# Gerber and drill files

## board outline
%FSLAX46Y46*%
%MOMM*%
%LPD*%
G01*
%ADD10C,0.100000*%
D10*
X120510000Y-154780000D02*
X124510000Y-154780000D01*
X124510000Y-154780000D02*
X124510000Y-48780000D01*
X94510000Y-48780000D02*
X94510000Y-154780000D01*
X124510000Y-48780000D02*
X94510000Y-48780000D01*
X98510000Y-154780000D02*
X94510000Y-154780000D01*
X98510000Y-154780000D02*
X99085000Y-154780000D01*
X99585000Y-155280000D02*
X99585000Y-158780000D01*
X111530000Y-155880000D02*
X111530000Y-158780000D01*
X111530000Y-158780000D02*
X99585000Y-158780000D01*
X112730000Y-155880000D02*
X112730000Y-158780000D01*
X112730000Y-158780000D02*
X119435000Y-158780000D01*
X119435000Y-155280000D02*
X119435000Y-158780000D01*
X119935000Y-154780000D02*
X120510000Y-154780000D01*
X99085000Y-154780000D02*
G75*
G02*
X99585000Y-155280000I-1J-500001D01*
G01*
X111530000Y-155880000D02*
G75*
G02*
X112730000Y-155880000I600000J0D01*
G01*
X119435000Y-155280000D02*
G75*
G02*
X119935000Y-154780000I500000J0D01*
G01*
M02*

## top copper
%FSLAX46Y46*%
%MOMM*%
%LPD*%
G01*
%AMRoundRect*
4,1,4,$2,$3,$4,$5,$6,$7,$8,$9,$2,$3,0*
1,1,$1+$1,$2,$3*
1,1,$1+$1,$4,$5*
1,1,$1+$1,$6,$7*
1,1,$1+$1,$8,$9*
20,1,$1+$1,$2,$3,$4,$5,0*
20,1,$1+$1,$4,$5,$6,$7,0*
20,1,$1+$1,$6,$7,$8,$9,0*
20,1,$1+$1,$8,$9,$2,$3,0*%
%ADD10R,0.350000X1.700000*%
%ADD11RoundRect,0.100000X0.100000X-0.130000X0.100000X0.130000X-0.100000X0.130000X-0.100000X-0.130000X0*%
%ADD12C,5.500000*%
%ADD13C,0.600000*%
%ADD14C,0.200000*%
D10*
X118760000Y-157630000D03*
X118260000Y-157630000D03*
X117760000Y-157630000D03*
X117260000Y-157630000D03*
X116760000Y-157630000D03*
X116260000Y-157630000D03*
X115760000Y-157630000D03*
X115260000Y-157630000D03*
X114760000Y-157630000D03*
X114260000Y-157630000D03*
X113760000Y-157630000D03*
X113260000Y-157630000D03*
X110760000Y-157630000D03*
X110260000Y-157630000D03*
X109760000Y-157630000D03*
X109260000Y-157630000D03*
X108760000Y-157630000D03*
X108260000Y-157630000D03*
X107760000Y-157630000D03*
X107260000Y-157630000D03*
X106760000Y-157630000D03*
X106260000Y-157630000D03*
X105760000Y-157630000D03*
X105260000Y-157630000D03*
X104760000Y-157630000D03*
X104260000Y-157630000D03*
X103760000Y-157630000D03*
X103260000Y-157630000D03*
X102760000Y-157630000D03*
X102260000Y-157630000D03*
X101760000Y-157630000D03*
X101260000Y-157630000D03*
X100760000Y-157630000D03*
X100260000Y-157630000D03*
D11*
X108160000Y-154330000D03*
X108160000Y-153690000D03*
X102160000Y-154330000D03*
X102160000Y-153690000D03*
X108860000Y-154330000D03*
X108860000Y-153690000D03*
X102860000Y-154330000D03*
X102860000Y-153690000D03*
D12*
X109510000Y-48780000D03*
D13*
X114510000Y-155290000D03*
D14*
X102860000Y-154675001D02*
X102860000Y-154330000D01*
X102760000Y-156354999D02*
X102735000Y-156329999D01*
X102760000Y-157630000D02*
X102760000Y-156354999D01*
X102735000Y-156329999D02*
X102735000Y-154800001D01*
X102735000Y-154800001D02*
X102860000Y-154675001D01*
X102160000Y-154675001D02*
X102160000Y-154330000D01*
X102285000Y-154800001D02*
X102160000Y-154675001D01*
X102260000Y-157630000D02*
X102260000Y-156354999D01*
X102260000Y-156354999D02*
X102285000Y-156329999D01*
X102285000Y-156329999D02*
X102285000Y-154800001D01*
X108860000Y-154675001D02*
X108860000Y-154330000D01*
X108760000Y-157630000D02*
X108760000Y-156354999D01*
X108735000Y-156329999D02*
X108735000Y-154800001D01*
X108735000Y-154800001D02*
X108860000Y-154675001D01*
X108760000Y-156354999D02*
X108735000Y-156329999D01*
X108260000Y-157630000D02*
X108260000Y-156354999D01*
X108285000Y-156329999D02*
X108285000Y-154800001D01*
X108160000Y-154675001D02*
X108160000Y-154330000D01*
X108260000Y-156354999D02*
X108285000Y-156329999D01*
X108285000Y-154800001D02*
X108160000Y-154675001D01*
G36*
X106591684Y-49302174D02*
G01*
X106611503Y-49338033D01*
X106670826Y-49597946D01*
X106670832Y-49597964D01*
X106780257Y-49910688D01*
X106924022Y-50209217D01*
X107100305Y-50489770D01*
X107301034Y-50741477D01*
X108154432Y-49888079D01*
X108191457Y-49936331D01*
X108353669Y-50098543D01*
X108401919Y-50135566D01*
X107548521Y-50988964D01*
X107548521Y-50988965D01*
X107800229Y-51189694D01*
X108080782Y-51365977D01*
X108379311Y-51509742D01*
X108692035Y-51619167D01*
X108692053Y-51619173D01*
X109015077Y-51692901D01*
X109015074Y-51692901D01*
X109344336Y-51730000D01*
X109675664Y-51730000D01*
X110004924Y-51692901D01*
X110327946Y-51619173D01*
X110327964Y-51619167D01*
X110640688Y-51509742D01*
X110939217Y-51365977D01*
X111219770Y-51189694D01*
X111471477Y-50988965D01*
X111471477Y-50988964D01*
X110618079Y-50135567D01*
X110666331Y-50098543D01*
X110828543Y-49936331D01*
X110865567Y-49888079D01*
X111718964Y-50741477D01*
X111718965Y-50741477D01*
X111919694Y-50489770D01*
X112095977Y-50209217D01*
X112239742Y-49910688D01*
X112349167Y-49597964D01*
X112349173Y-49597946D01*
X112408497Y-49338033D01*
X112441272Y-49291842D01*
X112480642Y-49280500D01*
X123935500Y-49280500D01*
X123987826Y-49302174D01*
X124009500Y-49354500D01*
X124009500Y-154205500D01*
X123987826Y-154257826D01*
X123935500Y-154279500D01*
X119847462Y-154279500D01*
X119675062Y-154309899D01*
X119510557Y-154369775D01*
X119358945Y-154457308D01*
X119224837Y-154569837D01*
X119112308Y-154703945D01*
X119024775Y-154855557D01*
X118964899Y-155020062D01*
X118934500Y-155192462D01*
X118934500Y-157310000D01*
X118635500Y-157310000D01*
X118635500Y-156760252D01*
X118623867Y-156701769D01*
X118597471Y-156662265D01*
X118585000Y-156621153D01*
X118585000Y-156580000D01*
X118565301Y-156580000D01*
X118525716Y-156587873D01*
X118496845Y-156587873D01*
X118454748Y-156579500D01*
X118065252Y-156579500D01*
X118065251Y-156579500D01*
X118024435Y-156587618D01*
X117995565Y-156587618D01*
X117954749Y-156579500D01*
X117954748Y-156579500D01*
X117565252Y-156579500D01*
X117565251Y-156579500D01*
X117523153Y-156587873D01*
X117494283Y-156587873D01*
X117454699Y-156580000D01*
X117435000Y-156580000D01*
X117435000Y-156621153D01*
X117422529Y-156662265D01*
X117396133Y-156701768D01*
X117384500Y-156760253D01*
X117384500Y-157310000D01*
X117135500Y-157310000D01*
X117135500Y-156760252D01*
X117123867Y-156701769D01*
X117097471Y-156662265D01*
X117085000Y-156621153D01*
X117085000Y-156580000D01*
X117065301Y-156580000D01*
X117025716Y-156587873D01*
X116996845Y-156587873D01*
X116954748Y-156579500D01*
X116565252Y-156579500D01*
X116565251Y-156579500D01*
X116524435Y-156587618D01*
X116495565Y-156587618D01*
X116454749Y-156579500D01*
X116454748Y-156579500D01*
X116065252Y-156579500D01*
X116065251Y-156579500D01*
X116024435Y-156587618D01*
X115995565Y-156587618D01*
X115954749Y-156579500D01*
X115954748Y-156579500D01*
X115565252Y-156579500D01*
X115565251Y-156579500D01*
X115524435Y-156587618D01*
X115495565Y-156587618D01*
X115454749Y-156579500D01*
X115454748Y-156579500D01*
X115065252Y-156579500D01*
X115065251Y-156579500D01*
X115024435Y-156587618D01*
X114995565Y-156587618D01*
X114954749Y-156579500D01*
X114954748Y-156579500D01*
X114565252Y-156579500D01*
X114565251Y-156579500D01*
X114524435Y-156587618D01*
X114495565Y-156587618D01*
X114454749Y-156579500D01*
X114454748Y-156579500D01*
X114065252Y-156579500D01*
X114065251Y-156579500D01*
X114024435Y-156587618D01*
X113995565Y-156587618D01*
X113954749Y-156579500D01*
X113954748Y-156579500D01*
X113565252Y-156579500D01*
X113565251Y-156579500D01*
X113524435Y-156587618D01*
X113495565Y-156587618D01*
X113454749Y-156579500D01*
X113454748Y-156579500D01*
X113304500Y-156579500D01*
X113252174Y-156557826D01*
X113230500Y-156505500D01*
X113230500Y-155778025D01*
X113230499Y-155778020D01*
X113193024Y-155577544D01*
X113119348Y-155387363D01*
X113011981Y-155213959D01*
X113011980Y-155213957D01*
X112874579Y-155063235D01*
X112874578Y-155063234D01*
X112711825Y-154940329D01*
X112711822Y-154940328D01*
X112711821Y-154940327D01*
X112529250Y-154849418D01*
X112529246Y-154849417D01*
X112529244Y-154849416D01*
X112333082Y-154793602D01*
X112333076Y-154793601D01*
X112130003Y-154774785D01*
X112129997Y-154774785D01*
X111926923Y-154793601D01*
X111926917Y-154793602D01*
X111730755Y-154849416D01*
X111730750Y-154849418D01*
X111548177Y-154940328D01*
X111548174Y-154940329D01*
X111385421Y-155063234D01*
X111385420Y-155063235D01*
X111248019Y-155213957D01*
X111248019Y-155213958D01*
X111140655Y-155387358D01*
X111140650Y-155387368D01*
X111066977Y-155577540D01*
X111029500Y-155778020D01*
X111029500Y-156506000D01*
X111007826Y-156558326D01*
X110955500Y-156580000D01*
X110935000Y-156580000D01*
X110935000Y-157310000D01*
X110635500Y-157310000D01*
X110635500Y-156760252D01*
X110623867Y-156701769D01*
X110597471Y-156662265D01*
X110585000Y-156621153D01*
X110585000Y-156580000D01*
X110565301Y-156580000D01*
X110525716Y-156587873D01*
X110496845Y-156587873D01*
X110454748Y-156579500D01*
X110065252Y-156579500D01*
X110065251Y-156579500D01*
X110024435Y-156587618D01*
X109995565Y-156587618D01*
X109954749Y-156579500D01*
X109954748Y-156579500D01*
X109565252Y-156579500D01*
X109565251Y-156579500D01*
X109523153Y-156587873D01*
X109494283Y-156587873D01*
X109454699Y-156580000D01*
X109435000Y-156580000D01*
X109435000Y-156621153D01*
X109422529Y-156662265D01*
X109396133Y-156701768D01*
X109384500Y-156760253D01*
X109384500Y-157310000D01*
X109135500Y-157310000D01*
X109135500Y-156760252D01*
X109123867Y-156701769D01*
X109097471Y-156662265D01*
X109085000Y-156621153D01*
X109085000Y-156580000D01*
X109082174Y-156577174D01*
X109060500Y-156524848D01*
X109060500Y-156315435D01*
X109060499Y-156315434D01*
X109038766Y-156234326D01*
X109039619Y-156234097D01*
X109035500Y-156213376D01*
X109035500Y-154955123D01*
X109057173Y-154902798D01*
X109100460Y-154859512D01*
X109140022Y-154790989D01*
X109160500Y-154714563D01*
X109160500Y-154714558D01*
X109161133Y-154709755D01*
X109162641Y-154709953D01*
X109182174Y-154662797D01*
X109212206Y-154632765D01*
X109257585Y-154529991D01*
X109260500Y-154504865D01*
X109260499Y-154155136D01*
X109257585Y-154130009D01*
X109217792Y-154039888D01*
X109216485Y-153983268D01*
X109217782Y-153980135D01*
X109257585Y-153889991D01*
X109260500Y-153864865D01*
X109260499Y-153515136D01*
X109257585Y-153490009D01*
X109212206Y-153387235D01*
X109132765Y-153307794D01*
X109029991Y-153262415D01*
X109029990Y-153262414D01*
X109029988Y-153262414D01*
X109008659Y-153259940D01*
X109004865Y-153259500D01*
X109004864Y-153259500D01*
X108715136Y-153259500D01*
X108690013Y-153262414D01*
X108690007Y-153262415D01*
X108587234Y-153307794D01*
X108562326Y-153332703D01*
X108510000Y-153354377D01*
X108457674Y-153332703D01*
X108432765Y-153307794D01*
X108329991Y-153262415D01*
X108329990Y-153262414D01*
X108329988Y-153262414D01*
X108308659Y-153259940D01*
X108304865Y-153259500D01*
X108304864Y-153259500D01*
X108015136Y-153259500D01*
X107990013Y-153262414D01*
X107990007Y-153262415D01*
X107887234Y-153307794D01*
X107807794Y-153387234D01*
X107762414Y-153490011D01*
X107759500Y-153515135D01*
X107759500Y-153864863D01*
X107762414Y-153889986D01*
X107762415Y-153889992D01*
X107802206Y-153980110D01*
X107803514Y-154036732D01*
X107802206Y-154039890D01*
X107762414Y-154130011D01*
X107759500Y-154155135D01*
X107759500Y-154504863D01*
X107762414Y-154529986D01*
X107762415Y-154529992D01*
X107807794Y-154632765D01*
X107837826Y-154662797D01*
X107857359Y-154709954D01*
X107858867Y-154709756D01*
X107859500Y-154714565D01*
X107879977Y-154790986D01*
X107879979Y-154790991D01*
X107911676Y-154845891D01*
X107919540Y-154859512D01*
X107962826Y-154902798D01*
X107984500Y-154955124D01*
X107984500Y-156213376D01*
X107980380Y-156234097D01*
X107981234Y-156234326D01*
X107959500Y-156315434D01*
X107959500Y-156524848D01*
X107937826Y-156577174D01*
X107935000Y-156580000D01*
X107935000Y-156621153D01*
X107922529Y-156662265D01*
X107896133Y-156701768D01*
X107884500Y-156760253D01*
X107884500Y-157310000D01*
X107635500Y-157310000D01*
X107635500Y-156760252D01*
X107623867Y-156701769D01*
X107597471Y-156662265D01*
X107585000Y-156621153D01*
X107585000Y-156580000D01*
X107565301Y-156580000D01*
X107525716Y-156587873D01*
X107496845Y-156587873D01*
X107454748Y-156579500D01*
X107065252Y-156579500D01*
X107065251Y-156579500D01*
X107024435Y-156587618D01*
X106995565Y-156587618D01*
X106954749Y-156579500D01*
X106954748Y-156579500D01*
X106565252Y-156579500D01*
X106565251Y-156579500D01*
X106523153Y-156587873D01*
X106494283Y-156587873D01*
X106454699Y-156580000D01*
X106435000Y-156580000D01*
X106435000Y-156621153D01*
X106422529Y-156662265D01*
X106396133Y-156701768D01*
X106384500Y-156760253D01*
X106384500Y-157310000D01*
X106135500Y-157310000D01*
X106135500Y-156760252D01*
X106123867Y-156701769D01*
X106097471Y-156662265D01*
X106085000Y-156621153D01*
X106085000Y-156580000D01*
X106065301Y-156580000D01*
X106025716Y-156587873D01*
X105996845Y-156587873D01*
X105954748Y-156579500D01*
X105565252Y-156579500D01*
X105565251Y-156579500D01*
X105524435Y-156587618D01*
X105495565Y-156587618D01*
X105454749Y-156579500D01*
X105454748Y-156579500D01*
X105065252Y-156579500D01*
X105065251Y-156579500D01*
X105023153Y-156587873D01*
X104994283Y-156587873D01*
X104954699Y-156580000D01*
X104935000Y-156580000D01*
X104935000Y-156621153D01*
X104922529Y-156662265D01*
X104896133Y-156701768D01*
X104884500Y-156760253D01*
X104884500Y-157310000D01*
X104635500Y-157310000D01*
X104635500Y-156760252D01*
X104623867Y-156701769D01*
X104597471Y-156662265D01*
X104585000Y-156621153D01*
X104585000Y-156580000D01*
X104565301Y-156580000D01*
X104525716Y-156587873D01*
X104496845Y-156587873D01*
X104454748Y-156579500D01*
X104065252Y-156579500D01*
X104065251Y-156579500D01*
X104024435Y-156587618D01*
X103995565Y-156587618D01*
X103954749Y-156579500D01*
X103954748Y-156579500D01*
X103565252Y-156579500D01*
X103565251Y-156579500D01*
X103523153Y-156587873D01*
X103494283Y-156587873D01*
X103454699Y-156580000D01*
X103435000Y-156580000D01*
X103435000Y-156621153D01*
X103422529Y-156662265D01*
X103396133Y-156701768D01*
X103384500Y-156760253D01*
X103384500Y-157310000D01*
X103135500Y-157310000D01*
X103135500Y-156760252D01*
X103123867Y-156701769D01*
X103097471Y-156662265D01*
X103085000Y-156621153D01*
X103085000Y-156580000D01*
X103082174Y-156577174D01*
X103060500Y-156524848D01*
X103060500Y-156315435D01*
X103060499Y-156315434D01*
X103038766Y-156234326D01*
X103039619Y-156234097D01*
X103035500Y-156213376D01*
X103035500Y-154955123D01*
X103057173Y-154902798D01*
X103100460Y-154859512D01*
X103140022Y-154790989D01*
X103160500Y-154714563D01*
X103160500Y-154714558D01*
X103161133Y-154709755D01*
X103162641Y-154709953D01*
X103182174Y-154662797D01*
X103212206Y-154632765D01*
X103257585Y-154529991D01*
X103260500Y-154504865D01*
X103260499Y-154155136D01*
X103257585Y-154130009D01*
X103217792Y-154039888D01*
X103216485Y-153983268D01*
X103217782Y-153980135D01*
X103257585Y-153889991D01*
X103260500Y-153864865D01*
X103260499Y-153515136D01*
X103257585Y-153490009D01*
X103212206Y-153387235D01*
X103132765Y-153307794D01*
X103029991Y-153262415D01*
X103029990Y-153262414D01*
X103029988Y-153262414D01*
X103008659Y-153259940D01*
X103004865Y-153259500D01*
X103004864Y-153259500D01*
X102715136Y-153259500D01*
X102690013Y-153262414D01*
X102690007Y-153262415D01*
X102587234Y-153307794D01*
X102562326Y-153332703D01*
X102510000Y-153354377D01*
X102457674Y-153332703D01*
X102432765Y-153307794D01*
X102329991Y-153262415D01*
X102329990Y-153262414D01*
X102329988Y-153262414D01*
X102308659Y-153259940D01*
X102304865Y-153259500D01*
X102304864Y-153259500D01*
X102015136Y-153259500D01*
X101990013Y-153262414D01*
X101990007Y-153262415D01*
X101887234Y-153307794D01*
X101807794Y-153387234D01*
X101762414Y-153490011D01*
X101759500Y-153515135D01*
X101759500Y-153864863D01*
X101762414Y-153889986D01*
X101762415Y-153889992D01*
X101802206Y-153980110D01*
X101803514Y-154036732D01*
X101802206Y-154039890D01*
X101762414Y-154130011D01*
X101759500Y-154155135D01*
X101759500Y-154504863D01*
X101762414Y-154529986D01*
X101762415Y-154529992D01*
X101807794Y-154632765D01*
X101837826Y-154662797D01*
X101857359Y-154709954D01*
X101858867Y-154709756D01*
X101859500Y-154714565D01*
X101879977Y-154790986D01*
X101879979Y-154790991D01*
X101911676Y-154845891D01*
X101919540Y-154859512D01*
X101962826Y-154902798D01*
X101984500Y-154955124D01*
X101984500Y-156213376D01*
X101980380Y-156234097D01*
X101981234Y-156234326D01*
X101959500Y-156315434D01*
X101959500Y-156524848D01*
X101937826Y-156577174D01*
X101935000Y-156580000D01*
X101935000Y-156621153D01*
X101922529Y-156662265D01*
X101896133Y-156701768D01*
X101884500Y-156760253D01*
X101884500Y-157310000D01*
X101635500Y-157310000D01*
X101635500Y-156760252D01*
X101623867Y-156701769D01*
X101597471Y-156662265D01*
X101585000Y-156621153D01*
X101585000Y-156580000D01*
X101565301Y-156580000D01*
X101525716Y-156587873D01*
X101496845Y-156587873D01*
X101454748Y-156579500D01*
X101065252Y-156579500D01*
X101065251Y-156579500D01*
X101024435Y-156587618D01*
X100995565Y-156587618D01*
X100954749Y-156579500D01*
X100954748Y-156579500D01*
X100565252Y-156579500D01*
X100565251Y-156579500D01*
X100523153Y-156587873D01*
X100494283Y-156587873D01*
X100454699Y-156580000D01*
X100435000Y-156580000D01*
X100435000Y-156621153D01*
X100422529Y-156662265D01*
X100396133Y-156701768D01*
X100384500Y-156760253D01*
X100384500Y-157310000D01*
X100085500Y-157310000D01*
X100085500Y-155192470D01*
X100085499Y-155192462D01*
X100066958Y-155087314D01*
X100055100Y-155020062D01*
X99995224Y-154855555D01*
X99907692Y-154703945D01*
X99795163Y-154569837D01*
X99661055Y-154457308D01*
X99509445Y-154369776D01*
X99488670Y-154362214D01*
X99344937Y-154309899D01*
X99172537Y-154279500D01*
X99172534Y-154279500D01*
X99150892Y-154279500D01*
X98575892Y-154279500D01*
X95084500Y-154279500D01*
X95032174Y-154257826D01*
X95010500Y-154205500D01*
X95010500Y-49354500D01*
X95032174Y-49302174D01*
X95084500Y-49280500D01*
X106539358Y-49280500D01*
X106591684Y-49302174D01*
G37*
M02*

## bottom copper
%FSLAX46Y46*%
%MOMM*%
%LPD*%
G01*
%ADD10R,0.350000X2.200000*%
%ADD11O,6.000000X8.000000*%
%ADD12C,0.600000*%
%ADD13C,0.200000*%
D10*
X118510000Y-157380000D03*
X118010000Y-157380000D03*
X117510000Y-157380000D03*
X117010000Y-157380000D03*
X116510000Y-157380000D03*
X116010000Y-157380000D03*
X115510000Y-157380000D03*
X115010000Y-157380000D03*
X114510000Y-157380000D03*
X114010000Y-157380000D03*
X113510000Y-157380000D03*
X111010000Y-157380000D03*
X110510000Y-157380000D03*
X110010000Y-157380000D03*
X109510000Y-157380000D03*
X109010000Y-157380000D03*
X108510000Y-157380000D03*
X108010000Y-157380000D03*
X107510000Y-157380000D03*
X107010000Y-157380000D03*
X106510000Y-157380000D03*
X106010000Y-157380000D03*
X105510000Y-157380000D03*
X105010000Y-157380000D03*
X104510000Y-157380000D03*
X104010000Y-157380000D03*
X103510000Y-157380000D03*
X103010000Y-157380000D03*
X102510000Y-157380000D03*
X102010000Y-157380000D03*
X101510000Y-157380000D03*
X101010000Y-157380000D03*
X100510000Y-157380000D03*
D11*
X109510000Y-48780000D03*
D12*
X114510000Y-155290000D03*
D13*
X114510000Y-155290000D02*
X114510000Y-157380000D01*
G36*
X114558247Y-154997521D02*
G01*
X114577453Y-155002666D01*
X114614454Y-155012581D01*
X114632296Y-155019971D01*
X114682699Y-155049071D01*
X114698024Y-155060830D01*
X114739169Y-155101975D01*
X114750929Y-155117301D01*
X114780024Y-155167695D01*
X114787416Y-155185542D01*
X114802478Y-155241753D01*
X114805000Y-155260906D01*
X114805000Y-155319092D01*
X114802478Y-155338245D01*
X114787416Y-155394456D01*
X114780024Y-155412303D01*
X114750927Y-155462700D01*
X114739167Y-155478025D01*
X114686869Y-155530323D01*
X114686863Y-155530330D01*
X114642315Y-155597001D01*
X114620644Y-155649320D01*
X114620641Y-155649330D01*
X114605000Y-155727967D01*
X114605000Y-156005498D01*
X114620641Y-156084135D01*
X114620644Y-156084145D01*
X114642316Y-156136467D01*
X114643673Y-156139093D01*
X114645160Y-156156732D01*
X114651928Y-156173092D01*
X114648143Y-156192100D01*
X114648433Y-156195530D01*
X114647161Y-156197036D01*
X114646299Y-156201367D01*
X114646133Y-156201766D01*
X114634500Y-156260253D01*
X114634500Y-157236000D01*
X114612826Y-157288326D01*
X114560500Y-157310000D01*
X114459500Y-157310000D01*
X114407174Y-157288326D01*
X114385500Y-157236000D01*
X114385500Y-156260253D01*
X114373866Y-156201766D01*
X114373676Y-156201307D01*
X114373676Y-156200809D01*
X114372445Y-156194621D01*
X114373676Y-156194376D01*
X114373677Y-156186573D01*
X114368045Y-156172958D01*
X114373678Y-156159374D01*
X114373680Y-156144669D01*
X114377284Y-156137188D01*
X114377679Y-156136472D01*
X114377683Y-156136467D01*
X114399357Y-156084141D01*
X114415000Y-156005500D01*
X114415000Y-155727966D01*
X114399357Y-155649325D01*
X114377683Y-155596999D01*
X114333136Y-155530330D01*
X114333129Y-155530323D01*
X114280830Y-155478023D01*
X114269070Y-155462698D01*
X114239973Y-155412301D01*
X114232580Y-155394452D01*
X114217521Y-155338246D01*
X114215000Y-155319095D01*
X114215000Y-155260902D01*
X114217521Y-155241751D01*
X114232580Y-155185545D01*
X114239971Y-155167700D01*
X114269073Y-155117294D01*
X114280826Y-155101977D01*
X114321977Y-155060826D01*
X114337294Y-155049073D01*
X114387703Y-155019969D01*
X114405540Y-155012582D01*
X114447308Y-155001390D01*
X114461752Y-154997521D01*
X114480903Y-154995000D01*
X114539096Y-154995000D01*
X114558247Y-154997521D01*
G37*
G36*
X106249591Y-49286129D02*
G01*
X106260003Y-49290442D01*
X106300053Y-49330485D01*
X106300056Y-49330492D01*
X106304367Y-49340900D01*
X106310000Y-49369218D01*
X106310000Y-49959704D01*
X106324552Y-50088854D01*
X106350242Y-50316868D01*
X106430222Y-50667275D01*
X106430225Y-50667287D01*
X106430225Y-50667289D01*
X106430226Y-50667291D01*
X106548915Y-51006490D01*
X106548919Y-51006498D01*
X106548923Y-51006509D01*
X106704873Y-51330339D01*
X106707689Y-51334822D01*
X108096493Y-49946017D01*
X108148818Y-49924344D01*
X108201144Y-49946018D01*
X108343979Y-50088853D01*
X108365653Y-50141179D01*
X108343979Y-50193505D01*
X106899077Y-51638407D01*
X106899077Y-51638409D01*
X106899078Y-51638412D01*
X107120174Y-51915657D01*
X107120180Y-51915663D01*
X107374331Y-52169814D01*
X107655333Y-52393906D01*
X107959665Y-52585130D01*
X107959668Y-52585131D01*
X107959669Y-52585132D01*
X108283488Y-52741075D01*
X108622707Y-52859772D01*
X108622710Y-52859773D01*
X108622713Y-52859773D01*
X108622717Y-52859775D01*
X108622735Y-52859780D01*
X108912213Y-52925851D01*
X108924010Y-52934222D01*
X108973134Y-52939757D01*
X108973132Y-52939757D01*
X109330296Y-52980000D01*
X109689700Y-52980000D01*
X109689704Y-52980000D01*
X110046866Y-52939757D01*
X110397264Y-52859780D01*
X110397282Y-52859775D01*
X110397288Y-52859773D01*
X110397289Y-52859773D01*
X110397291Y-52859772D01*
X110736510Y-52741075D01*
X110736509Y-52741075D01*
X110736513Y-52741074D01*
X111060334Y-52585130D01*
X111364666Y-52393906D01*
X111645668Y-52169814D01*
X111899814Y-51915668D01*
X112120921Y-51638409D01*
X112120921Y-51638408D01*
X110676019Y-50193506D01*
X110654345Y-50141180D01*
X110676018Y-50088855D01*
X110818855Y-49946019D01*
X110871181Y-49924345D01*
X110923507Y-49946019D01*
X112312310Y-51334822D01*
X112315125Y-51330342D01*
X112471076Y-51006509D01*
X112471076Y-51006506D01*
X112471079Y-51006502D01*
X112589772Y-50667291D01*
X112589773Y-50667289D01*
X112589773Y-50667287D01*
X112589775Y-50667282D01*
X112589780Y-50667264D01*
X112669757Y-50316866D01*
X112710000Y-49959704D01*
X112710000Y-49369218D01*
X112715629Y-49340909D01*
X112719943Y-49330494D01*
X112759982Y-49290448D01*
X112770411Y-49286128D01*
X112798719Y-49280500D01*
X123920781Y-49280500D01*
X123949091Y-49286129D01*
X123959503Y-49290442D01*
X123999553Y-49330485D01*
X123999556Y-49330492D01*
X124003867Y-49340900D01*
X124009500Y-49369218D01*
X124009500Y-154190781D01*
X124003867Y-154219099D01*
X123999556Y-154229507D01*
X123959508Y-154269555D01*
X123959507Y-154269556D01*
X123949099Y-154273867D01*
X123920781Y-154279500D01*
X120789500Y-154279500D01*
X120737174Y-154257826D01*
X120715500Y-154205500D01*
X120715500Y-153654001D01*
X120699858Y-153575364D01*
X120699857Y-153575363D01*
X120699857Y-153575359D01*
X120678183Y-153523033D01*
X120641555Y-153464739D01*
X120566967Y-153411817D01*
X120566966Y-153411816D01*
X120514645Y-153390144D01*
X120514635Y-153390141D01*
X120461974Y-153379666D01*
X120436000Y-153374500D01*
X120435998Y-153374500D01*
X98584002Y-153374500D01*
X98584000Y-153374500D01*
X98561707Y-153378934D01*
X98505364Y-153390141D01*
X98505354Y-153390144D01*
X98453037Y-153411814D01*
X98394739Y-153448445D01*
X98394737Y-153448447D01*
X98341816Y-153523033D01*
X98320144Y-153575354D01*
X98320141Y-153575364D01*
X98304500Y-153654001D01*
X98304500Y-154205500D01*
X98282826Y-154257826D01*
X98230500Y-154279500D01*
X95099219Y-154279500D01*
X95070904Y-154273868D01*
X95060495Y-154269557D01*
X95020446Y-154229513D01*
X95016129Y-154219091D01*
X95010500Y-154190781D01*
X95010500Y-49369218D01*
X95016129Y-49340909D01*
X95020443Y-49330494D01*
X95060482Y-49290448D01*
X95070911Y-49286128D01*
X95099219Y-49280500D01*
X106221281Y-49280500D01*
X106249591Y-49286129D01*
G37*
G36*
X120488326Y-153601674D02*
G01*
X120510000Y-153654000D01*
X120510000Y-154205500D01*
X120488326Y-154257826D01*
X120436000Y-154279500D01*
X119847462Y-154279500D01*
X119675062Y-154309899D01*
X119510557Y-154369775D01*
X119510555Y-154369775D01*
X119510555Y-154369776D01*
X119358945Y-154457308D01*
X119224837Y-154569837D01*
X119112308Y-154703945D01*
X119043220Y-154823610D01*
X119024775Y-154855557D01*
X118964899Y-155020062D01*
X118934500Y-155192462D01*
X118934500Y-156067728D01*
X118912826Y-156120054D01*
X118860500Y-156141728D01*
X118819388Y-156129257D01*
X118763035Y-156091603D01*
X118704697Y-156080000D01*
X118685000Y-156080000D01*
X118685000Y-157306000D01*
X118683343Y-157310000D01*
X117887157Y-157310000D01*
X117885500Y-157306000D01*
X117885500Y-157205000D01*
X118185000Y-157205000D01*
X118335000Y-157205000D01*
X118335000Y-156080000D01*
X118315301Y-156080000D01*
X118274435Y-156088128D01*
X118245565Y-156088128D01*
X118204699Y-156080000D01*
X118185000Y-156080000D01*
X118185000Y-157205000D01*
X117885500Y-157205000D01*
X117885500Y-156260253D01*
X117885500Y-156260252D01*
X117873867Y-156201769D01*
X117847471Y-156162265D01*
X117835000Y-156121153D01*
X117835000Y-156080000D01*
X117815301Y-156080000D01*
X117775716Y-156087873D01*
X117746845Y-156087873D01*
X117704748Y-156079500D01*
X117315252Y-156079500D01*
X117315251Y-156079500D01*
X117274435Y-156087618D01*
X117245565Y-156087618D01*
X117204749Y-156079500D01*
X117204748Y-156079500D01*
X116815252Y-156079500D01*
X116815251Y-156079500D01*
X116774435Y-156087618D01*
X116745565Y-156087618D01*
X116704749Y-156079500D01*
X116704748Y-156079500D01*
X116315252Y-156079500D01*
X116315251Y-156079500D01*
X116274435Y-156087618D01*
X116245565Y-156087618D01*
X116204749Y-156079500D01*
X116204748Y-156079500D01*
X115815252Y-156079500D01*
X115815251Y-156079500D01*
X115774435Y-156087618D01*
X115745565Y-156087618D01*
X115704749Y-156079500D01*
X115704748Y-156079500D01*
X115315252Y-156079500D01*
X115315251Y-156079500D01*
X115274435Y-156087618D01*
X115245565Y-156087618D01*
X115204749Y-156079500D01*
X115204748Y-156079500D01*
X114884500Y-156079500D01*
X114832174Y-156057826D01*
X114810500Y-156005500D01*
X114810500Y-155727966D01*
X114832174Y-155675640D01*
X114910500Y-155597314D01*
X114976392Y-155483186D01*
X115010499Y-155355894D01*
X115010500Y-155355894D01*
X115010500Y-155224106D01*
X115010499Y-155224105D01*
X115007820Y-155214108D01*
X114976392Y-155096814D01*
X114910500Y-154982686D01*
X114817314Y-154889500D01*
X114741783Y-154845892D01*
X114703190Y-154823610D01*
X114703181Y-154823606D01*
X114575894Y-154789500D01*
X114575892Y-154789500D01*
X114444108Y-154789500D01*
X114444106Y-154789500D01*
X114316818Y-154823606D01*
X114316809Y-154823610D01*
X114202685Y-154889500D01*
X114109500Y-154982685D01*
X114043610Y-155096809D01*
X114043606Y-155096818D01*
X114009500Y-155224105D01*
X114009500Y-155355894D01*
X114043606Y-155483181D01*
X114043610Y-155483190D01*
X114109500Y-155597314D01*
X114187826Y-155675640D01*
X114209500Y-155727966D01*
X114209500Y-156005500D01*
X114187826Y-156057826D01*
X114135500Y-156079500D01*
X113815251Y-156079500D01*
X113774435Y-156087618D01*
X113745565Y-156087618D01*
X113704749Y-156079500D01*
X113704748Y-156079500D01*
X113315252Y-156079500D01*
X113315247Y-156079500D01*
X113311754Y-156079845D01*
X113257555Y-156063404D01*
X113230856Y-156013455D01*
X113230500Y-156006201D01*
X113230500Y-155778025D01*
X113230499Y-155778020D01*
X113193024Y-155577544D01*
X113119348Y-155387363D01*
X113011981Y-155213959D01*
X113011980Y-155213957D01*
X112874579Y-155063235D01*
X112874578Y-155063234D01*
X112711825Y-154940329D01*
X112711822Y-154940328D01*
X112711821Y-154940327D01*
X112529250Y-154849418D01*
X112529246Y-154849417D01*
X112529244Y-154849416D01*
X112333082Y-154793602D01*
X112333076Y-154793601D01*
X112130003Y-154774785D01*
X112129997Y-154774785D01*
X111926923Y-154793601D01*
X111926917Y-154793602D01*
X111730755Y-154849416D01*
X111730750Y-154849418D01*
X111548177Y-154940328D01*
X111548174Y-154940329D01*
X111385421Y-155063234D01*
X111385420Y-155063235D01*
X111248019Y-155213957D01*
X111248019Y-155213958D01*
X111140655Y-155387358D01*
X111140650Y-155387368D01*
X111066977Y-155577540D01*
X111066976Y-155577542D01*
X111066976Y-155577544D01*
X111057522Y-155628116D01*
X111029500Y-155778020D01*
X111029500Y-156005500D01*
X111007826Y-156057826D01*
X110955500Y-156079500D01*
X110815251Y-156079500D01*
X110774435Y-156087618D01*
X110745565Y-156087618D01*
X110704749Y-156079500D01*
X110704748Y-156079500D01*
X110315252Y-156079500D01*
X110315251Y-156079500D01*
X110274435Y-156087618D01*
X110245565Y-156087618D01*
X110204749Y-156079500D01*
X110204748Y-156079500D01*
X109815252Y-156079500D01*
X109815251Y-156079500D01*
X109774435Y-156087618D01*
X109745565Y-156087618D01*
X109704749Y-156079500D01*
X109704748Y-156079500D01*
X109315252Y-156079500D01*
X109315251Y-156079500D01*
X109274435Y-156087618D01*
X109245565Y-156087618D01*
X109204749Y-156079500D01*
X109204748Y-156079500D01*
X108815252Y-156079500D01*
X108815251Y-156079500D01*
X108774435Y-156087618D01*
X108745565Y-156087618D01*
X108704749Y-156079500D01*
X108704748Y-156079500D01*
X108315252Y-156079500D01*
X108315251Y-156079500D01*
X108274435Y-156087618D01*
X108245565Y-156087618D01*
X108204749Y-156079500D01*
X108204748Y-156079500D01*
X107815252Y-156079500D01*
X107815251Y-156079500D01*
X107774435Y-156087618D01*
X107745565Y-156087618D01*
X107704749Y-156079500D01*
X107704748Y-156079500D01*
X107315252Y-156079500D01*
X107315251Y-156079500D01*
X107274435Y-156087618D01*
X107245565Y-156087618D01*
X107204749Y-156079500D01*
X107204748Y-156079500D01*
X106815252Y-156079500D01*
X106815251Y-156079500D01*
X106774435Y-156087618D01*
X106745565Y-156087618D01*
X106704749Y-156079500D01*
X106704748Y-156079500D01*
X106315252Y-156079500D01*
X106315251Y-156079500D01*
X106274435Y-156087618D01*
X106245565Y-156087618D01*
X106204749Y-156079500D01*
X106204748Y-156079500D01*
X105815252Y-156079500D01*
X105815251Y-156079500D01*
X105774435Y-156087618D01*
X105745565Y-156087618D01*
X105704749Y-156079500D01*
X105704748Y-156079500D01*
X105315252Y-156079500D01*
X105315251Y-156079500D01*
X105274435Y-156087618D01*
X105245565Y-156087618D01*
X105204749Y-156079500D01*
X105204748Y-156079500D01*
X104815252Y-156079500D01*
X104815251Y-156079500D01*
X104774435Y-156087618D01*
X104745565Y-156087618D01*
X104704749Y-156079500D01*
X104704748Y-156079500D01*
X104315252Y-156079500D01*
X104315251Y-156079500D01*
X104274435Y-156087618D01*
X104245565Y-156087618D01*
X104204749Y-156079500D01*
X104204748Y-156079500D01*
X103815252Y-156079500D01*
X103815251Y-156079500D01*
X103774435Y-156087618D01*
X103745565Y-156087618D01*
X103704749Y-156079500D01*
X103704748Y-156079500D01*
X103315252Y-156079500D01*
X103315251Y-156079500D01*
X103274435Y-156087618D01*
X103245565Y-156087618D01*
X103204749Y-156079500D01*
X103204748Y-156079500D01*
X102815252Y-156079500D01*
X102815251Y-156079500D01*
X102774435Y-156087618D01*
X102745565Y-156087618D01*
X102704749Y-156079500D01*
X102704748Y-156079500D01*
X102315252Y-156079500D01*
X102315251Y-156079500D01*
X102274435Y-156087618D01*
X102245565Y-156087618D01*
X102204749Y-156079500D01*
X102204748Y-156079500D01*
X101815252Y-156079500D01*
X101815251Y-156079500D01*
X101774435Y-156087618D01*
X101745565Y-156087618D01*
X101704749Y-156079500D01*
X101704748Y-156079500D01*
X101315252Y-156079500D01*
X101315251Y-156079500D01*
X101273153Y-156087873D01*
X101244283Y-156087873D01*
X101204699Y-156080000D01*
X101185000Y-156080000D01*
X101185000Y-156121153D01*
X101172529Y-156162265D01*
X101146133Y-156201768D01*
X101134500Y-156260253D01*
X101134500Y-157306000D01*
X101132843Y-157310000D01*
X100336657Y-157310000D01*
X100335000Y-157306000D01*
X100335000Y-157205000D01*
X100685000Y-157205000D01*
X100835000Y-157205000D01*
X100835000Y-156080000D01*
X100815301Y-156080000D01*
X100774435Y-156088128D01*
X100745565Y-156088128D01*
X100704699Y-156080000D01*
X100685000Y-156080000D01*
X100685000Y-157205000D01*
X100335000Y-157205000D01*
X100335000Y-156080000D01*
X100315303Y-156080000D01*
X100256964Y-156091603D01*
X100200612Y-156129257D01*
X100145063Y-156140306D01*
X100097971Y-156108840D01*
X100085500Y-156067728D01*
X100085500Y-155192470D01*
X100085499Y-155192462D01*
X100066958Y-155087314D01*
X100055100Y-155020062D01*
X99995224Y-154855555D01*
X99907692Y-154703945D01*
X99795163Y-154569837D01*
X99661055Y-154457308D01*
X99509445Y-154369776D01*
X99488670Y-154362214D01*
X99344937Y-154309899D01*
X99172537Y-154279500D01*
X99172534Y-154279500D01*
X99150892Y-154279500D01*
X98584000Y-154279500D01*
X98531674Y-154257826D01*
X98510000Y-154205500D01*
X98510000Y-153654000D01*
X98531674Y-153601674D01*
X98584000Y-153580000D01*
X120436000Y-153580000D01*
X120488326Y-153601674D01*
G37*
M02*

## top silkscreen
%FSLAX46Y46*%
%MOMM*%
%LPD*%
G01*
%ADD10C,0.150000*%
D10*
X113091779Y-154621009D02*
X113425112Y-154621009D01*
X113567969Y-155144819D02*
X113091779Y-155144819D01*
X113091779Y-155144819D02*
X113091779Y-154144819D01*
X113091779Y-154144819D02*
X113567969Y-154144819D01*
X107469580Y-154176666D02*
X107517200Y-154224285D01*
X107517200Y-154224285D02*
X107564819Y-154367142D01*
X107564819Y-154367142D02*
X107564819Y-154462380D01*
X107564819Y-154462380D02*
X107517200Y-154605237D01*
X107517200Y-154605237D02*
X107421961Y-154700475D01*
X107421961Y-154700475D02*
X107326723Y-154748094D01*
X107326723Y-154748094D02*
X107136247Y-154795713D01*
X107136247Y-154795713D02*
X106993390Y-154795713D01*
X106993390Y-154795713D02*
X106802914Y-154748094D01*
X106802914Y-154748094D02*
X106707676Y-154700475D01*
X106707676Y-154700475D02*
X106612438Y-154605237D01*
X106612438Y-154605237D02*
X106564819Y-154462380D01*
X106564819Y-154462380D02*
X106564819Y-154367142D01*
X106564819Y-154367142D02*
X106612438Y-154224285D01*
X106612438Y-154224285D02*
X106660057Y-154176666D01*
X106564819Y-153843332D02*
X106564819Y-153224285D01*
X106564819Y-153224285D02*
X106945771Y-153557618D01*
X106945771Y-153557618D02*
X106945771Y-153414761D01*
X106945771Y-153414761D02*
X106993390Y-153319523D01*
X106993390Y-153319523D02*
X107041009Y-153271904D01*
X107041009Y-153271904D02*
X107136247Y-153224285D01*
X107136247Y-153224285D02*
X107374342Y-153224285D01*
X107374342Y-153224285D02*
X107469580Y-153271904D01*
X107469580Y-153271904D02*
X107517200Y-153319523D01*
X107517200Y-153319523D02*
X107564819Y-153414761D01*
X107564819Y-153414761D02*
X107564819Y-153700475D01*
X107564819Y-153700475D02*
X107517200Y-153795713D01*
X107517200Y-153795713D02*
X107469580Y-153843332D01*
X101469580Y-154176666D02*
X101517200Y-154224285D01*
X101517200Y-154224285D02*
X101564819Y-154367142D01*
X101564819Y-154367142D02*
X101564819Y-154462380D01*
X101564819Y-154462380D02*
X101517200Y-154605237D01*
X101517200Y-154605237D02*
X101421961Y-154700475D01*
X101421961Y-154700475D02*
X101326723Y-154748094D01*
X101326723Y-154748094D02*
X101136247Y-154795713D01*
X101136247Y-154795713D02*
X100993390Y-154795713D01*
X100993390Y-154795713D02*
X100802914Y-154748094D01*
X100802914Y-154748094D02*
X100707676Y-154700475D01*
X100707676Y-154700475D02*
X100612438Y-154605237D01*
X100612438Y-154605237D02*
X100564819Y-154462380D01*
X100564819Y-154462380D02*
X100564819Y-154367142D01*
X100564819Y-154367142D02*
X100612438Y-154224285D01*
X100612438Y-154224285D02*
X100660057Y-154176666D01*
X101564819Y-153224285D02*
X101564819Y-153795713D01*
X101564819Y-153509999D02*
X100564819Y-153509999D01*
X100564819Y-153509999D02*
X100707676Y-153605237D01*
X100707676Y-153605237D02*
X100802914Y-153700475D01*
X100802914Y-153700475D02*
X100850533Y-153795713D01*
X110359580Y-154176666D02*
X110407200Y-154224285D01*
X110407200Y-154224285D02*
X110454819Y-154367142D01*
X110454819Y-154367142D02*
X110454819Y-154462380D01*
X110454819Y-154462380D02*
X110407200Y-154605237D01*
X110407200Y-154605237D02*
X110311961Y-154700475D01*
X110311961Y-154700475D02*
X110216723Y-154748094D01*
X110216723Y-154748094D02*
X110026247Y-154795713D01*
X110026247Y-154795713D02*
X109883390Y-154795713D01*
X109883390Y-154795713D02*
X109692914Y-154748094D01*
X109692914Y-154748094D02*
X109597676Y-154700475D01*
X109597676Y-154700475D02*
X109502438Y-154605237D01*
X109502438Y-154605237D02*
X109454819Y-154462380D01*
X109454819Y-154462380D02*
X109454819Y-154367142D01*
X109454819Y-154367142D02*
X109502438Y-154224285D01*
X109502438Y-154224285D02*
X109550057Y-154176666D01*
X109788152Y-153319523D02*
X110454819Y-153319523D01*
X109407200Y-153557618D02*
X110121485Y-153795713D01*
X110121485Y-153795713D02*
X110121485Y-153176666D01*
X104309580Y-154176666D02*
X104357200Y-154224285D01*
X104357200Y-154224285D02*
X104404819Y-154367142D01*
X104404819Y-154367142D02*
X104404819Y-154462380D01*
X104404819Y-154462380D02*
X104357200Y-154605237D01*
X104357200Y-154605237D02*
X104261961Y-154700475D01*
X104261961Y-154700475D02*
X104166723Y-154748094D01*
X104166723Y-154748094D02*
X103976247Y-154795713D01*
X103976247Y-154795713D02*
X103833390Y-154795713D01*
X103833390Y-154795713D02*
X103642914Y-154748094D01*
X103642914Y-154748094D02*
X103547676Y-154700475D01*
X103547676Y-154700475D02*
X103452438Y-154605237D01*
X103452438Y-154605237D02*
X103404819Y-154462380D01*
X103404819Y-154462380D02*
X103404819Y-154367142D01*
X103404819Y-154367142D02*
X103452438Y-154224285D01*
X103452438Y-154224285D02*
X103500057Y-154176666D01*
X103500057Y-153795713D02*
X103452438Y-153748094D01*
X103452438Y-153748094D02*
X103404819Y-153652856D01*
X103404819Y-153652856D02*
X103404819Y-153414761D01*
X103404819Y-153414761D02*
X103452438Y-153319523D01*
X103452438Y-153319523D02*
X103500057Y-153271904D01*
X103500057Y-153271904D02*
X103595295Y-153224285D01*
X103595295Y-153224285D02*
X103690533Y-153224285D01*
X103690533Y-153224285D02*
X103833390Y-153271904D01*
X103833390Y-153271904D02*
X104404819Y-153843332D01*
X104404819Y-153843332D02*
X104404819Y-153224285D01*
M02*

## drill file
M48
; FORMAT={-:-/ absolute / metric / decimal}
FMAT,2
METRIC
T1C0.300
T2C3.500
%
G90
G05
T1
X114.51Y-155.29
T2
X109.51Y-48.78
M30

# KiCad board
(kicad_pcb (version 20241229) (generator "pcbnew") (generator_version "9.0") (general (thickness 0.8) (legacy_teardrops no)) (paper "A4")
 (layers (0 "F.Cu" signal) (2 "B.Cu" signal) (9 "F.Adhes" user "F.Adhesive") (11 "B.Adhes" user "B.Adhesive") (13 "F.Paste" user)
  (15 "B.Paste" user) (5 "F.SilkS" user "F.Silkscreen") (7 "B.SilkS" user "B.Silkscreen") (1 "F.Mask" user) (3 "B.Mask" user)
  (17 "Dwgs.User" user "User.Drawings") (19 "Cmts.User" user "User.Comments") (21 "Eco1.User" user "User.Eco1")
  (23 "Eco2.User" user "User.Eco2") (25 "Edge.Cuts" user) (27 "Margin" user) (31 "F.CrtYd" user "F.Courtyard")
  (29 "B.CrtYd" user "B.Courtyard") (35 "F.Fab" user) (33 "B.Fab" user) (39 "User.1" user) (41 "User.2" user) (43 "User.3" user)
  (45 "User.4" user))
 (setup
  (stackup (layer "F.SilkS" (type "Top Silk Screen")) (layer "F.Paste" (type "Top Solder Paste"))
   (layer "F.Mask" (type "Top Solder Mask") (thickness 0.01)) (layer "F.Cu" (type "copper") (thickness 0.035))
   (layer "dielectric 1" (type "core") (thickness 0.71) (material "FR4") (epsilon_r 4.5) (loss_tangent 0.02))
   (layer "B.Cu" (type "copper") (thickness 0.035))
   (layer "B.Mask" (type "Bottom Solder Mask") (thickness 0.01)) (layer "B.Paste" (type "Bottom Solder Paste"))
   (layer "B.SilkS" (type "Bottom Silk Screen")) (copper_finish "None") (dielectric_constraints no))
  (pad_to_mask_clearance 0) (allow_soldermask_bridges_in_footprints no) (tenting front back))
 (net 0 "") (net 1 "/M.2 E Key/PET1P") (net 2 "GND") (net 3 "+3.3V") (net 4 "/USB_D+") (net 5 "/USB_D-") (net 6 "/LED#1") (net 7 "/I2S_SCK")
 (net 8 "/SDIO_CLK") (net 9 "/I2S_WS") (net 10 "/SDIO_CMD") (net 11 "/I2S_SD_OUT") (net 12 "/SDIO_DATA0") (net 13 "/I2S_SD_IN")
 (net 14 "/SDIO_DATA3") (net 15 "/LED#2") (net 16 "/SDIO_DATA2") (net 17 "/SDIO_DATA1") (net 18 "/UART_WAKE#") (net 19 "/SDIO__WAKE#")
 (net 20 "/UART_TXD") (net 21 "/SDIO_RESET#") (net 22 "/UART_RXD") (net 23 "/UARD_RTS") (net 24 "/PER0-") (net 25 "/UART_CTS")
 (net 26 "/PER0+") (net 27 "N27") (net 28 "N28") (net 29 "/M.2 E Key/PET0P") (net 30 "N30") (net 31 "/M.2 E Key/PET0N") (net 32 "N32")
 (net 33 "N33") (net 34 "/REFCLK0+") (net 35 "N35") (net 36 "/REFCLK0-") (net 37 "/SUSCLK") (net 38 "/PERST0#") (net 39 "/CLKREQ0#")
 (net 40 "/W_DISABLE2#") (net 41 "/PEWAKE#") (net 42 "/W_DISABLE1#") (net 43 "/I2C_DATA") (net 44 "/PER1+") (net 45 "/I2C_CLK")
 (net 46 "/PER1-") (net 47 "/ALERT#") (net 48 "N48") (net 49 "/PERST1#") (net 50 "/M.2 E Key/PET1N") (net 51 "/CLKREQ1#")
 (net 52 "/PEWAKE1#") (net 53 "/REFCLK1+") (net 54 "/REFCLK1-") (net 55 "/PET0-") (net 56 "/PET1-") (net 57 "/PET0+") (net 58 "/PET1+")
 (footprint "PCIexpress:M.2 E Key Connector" (layer "F.Cu") (at 109.51 157.67)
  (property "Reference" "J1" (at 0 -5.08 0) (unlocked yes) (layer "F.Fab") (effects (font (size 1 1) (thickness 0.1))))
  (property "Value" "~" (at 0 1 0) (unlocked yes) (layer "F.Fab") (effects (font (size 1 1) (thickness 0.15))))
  (fp_line (start -11 -2.89) (end -10.425 -2.89) (stroke (width 0.1) (type default)) (layer "Edge.Cuts") (net 1))
  (fp_line (start -9.925 -2.39) (end -9.925 1.11) (stroke (width 0.1) (type default)) (layer "Edge.Cuts") (net 1))
  (fp_line (start 2.02 -1.79) (end 2.02 1.11) (stroke (width 0.1) (type default)) (layer "Edge.Cuts") (net 1))
  (fp_line (start 2.02 1.11) (end -9.925 1.11) (stroke (width 0.1) (type default)) (layer "Edge.Cuts") (net 1))
  (fp_line (start 3.22 -1.79) (end 3.22 1.11) (stroke (width 0.1) (type default)) (layer "Edge.Cuts") (net 1))
  (fp_line (start 3.22 1.11) (end 9.925 1.11) (stroke (width 0.1) (type default)) (layer "Edge.Cuts") (net 1))
  (fp_line (start 9.925 -2.39) (end 9.925 1.11) (stroke (width 0.1) (type default)) (layer "Edge.Cuts") (net 1))
  (fp_line (start 10.425 -2.89) (end 11 -2.89) (stroke (width 0.1) (type default)) (layer "Edge.Cuts") (net 1))
  (fp_arc (start -10.425 -2.89) (mid -10.071447 -2.743553) (end -9.925 -2.39) (stroke (width 0.1) (type default)) (layer "Edge.Cuts")
   (net 1))
  (fp_arc (start 2.02 -1.79) (mid 2.62 -2.39) (end 3.22 -1.79) (stroke (width 0.1) (type default)) (layer "Edge.Cuts") (net 1))
  (fp_arc (start 9.925 -2.39) (mid 10.071447 -2.743553) (end 10.425 -2.89) (stroke (width 0.1) (type default)) (layer "Edge.Cuts") (net 1))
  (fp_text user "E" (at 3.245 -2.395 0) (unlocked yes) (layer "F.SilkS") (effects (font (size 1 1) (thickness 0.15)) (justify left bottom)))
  (pad "1" smd rect (at 9.25 -0.04 180) (size 0.35 1.7) (layers "F.Cu") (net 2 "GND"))
  (pad "2" smd rect (at 9 -0.29 180) (size 0.35 2.2) (layers "B.Cu") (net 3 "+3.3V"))
  (pad "3" smd rect (at 8.75 -0.04 180) (size 0.35 1.7) (layers "F.Cu") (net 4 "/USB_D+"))
  (pad "4" smd rect (at 8.5 -0.29 180) (size 0.35 2.2) (layers "B.Cu") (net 3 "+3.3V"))
  (pad "5" smd rect (at 8.25 -0.04 180) (size 0.35 1.7) (layers "F.Cu") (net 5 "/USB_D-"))
  (pad "6" smd rect (at 8 -0.29 180) (size 0.35 2.2) (layers "B.Cu") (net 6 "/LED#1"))
  (pad "7" smd rect (at 7.75 -0.04 180) (size 0.35 1.7) (layers "F.Cu") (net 2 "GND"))
  (pad "8" smd rect (at 7.5 -0.29 180) (size 0.35 2.2) (layers "B.Cu") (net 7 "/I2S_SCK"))
  (pad "9" smd rect (at 7.25 -0.04 180) (size 0.35 1.7) (layers "F.Cu") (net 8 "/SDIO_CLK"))
  (pad "10" smd rect (at 7 -0.29 180) (size 0.35 2.2) (layers "B.Cu") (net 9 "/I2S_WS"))
  (pad "11" smd rect (at 6.75 -0.04 180) (size 0.35 1.7) (layers "F.Cu") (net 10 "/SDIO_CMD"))
  (pad "12" smd rect (at 6.5 -0.29 180) (size 0.35 2.2) (layers "B.Cu") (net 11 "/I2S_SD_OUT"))
  (pad "13" smd rect (at 6.25 -0.04 180) (size 0.35 1.7) (layers "F.Cu") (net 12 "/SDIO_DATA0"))
  (pad "14" smd rect (at 6 -0.29 180) (size 0.35 2.2) (layers "B.Cu") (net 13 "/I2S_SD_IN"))
  (pad "15" smd rect (at 5.75 -0.04 180) (size 0.35 1.7) (layers "F.Cu") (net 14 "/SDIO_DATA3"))
  (pad "16" smd rect (at 5.5 -0.29 180) (size 0.35 2.2) (layers "B.Cu") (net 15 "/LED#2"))
  (pad "17" smd rect (at 5.25 -0.04 180) (size 0.35 1.7) (layers "F.Cu") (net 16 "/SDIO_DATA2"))
  (pad "18" smd rect (at 5 -0.29 180) (size 0.35 2.2) (layers "B.Cu") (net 2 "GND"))
  (pad "19" smd rect (at 4.75 -0.04 180) (size 0.35 1.7) (layers "F.Cu") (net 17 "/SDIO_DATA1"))
  (pad "20" smd rect (at 4.5 -0.29 180) (size 0.35 2.2) (layers "B.Cu") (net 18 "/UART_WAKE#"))
  (pad "21" smd rect (at 4.25 -0.04 180) (size 0.35 1.7) (layers "F.Cu") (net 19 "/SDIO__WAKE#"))
  (pad "22" smd rect (at 4 -0.29 180) (size 0.35 2.2) (layers "B.Cu") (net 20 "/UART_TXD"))
  (pad "23" smd rect (at 3.75 -0.04 180) (size 0.35 1.7) (layers "F.Cu") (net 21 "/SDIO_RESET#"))
  (pad "32" smd rect (at 1.5 -0.29 180) (size 0.35 2.2) (layers "B.Cu") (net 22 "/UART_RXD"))
  (pad "33" smd rect (at 1.25 -0.04 180) (size 0.35 1.7) (layers "F.Cu") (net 2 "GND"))
  (pad "34" smd rect (at 1 -0.29 180) (size 0.35 2.2) (layers "B.Cu") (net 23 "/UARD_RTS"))
  (pad "35" smd rect (at 0.75 -0.04 180) (size 0.35 1.7) (layers "F.Cu") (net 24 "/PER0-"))
  (pad "36" smd rect (at 0.5 -0.29 180) (size 0.35 2.2) (layers "B.Cu") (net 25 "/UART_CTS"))
  (pad "37" smd rect (at 0.25 -0.04 180) (size 0.35 1.7) (layers "F.Cu") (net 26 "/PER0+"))
  (pad "38" smd rect (at 0 -0.29 180) (size 0.35 2.2) (layers "B.Cu") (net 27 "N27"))
  (pad "39" smd rect (at -0.25 -0.04 180) (size 0.35 1.7) (layers "F.Cu") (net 2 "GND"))
  (pad "40" smd rect (at -0.5 -0.29 180) (size 0.35 2.2) (layers "B.Cu") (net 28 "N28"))
  (pad "41" smd rect (at -0.75 -0.04 180) (size 0.35 1.7) (layers "F.Cu") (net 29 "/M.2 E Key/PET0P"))
  (pad "42" smd rect (at -1 -0.29 180) (size 0.35 2.2) (layers "B.Cu") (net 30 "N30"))
  (pad "43" smd rect (at -1.25 -0.04 180) (size 0.35 1.7) (layers "F.Cu") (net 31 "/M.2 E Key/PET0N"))
  (pad "44" smd rect (at -1.5 -0.29 180) (size 0.35 2.2) (layers "B.Cu") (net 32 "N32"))
  (pad "45" smd rect (at -1.75 -0.04 180) (size 0.35 1.7) (layers "F.Cu") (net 2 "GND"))
  (pad "46" smd rect (at -2 -0.29 180) (size 0.35 2.2) (layers "B.Cu") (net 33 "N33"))
  (pad "47" smd rect (at -2.25 -0.04 180) (size 0.35 1.7) (layers "F.Cu") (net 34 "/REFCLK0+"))
  (pad "48" smd rect (at -2.5 -0.29 180) (size 0.35 2.2) (layers "B.Cu") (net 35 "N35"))
  (pad "49" smd rect (at -2.75 -0.04 180) (size 0.35 1.7) (layers "F.Cu") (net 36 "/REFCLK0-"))
  (pad "50" smd rect (at -3 -0.29 180) (size 0.35 2.2) (layers "B.Cu") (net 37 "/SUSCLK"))
  (pad "51" smd rect (at -3.25 -0.04 180) (size 0.35 1.7) (layers "F.Cu") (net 2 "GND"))
  (pad "52" smd rect (at -3.5 -0.29 180) (size 0.35 2.2) (layers "B.Cu") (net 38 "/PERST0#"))
  (pad "53" smd rect (at -3.75 -0.04 180) (size 0.35 1.7) (layers "F.Cu") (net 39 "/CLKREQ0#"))
  (pad "54" smd rect (at -4 -0.29 180) (size 0.35 2.2) (layers "B.Cu") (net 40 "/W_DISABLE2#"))
  (pad "55" smd rect (at -4.25 -0.04 180) (size 0.35 1.7) (layers "F.Cu") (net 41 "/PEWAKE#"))
  (pad "56" smd rect (at -4.5 -0.29 180) (size 0.35 2.2) (layers "B.Cu") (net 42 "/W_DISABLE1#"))
  (pad "57" smd rect (at -4.75 -0.04 180) (size 0.35 1.7) (layers "F.Cu") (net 2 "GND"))
  (pad "58" smd rect (at -5 -0.29 180) (size 0.35 2.2) (layers "B.Cu") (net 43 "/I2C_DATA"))
  (pad "59" smd rect (at -5.25 -0.04 180) (size 0.35 1.7) (layers "F.Cu") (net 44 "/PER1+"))
  (pad "60" smd rect (at -5.5 -0.29 180) (size 0.35 2.2) (layers "B.Cu") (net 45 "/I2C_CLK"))
  (pad "61" smd rect (at -5.75 -0.04 180) (size 0.35 1.7) (layers "F.Cu") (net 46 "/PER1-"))
  (pad "62" smd rect (at -6 -0.29 180) (size 0.35 2.2) (layers "B.Cu") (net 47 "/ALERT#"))
  (pad "63" smd rect (at -6.25 -0.04 180) (size 0.35 1.7) (layers "F.Cu") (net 2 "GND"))
  (pad "64" smd rect (at -6.5 -0.29 180) (size 0.35 2.2) (layers "B.Cu") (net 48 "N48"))
  (pad "65" smd rect (at -6.75 -0.04 180) (size 0.35 1.7) (layers "F.Cu") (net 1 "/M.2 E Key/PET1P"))
  (pad "66" smd rect (at -7 -0.29 180) (size 0.35 2.2) (layers "B.Cu") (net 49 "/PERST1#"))
  (pad "67" smd rect (at -7.25 -0.04 180) (size 0.35 1.7) (layers "F.Cu") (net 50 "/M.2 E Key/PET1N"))
  (pad "68" smd rect (at -7.5 -0.29 180) (size 0.35 2.2) (layers "B.Cu") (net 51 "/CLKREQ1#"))
  (pad "69" smd rect (at -7.75 -0.04 180) (size 0.35 1.7) (layers "F.Cu") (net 2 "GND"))
  (pad "70" smd rect (at -8 -0.29 180) (size 0.35 2.2) (layers "B.Cu") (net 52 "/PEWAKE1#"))
  (pad "71" smd rect (at -8.25 -0.04 180) (size 0.35 1.7) (layers "F.Cu") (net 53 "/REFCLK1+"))
  (pad "72" smd rect (at -8.5 -0.29 180) (size 0.35 2.2) (layers "B.Cu") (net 3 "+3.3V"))
  (pad "73" smd rect (at -8.75 -0.04 180) (size 0.35 1.7) (layers "F.Cu") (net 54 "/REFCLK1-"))
  (pad "74" smd rect (at -9 -0.29 180) (size 0.35 2.2) (layers "B.Cu") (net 3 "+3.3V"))
  (pad "75" smd rect (at -9.25 -0.04 180) (size 0.35 1.7) (layers "F.Cu") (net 2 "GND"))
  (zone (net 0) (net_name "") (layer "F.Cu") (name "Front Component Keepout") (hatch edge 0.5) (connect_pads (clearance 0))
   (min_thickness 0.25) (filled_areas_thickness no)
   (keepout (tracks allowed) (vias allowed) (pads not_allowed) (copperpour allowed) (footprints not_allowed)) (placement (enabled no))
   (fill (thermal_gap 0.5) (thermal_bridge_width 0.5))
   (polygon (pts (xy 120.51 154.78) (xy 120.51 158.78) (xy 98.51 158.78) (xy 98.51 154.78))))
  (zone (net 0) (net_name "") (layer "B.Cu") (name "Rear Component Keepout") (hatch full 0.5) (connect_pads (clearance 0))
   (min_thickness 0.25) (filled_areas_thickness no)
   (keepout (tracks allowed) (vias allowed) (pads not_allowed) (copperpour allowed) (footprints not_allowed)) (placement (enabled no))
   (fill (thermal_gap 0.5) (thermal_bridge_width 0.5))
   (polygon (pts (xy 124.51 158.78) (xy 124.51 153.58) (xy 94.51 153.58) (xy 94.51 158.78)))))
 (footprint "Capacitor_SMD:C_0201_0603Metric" (layer "F.Cu") (at 108.16 154.01 90)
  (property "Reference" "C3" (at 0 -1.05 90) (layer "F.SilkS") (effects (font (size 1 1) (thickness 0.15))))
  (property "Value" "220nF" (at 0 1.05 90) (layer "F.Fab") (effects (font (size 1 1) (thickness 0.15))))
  (pad "" smd roundrect (at -0.345 0 90) (size 0.318 0.36) (layers "F.Paste") (roundrect_rratio 0.25))
  (pad "" smd roundrect (at 0.345 0 90) (size 0.318 0.36) (layers "F.Paste") (roundrect_rratio 0.25))
  (pad "1" smd roundrect (at -0.32 0 90) (size 0.46 0.4) (layers "F.Cu" "F.Mask") (roundrect_rratio 0.25) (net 31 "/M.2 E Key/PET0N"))
  (pad "2" smd roundrect (at 0.32 0 90) (size 0.46 0.4) (layers "F.Cu" "F.Mask") (roundrect_rratio 0.25) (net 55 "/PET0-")))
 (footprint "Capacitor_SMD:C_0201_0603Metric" (layer "F.Cu") (at 102.16 154.01 90)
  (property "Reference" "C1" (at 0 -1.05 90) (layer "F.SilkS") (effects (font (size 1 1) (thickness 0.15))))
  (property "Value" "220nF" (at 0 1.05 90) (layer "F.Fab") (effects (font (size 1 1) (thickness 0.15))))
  (pad "" smd roundrect (at -0.345 0 90) (size 0.318 0.36) (layers "F.Paste") (roundrect_rratio 0.25))
  (pad "" smd roundrect (at 0.345 0 90) (size 0.318 0.36) (layers "F.Paste") (roundrect_rratio 0.25))
  (pad "1" smd roundrect (at -0.32 0 90) (size 0.46 0.4) (layers "F.Cu" "F.Mask") (roundrect_rratio 0.25) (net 50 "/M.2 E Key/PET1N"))
  (pad "2" smd roundrect (at 0.32 0 90) (size 0.46 0.4) (layers "F.Cu" "F.Mask") (roundrect_rratio 0.25) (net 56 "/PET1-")))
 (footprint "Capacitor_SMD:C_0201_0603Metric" (layer "F.Cu") (at 108.86 154.01 90)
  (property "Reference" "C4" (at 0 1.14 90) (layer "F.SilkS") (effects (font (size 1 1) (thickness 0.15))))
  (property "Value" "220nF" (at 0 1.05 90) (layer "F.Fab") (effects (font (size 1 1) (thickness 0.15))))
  (pad "" smd roundrect (at -0.345 0 90) (size 0.318 0.36) (layers "F.Paste") (roundrect_rratio 0.25))
  (pad "" smd roundrect (at 0.345 0 90) (size 0.318 0.36) (layers "F.Paste") (roundrect_rratio 0.25))
  (pad "1" smd roundrect (at -0.32 0 90) (size 0.46 0.4) (layers "F.Cu" "F.Mask") (roundrect_rratio 0.25) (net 29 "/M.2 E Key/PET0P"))
  (pad "2" smd roundrect (at 0.32 0 90) (size 0.46 0.4) (layers "F.Cu" "F.Mask") (roundrect_rratio 0.25) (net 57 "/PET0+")))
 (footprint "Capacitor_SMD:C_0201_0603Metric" (layer "F.Cu") (at 102.86 154.01 90)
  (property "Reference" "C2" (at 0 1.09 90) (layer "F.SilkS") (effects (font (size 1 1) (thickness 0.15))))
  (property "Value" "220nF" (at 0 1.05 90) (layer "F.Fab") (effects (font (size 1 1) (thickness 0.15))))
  (pad "" smd roundrect (at -0.345 0 90) (size 0.318 0.36) (layers "F.Paste") (roundrect_rratio 0.25))
  (pad "" smd roundrect (at 0.345 0 90) (size 0.318 0.36) (layers "F.Paste") (roundrect_rratio 0.25))
  (pad "1" smd roundrect (at -0.32 0 90) (size 0.46 0.4) (layers "F.Cu" "F.Mask") (roundrect_rratio 0.25) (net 1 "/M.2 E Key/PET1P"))
  (pad "2" smd roundrect (at 0.32 0 90) (size 0.46 0.4) (layers "F.Cu" "F.Mask") (roundrect_rratio 0.25) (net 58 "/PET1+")))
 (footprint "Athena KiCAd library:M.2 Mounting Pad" (layer "F.Cu") (at 109.51 48.78)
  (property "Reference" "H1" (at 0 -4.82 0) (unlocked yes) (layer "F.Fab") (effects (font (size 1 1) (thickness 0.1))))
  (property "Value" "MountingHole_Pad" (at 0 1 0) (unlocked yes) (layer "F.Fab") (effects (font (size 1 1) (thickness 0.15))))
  (pad "1" thru_hole circle (at 0 0) (size 5.5 5.5) (drill 3.5) (layers "*.Cu" "*.Mask") (remove_unused_layers no) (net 2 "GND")
   (padstack (mode front_inner_back)
    (layer "Inner" (shape circle) (size 5.5 5.5) (zone_connect -1))
    (layer "B.Cu" (shape oval) (size 6 8) (thermal_bridge_angle 45) (zone_connect -1)))))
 (gr_line (start 120.51 154.78) (end 124.51 154.78) (stroke (width 0.1) (type default)) (layer "Edge.Cuts"))
 (gr_line (start 124.51 154.78) (end 124.51 48.78) (stroke (width 0.1) (type default)) (layer "Edge.Cuts"))
 (gr_line (start 94.51 48.78) (end 94.51 154.78) (stroke (width 0.1) (type default)) (layer "Edge.Cuts"))
 (gr_line (start 124.51 48.78) (end 94.51 48.78) (stroke (width 0.1) (type default)) (layer "Edge.Cuts"))
 (gr_line (start 98.51 154.78) (end 94.51 154.78) (stroke (width 0.1) (type default)) (layer "Edge.Cuts"))
 (segment (start 102.86 154.675001) (end 102.86 154.33) (width 0.2) (layer "F.Cu") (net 1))
 (segment (start 102.76 156.354999) (end 102.735 156.329999) (width 0.2) (layer "F.Cu") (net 1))
 (segment (start 102.76 157.63) (end 102.76 156.354999) (width 0.2) (layer "F.Cu") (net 1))
 (segment (start 102.735 156.329999) (end 102.735 154.800001) (width 0.2) (layer "F.Cu") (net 1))
 (segment (start 102.735 154.800001) (end 102.86 154.675001) (width 0.2) (layer "F.Cu") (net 1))
 (segment (start 102.16 154.675001) (end 102.16 154.33) (width 0.2) (layer "F.Cu") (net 50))
 (segment (start 102.285 154.800001) (end 102.16 154.675001) (width 0.2) (layer "F.Cu") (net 50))
 (segment (start 102.26 157.63) (end 102.26 156.354999) (width 0.2) (layer "F.Cu") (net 50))
 (segment (start 102.26 156.354999) (end 102.285 156.329999) (width 0.2) (layer "F.Cu") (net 50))
 (segment (start 102.285 156.329999) (end 102.285 154.800001) (width 0.2) (layer "F.Cu") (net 50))
 (segment (start 108.86 154.675001) (end 108.86 154.33) (width 0.2) (layer "F.Cu") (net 29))
 (segment (start 108.76 157.63) (end 108.76 156.354999) (width 0.2) (layer "F.Cu") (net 29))
 (segment (start 108.735 156.329999) (end 108.735 154.800001) (width 0.2) (layer "F.Cu") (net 29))
 (segment (start 108.735 154.800001) (end 108.86 154.675001) (width 0.2) (layer "F.Cu") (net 29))
 (segment (start 108.76 156.354999) (end 108.735 156.329999) (width 0.2) (layer "F.Cu") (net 29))
 (segment (start 108.26 157.63) (end 108.26 156.354999) (width 0.2) (layer "F.Cu") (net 31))
 (segment (start 108.285 156.329999) (end 108.285 154.800001) (width 0.2) (layer "F.Cu") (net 31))
 (segment (start 108.16 154.675001) (end 108.16 154.33) (width 0.2) (layer "F.Cu") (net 31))
 (segment (start 108.26 156.354999) (end 108.285 156.329999) (width 0.2) (layer "F.Cu") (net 31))
 (segment (start 108.285 154.800001) (end 108.16 154.675001) (width 0.2) (layer "F.Cu") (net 31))
 (via (at 114.51 155.29) (size 0.6) (drill 0.3) (layers "F.Cu" "B.Cu") (free yes) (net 2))
 (segment (start 114.51 155.29) (end 114.51 157.38) (width 0.2) (layer "B.Cu") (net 2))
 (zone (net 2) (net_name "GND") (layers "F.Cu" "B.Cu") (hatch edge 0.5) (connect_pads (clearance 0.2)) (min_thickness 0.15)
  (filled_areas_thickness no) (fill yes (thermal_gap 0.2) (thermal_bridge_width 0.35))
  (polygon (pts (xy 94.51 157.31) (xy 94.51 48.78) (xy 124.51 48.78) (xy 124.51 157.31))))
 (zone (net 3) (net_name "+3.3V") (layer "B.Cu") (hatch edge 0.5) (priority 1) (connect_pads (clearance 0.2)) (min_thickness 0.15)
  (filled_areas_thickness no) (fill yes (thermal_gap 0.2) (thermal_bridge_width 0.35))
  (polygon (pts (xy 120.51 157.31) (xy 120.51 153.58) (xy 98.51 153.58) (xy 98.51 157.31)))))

